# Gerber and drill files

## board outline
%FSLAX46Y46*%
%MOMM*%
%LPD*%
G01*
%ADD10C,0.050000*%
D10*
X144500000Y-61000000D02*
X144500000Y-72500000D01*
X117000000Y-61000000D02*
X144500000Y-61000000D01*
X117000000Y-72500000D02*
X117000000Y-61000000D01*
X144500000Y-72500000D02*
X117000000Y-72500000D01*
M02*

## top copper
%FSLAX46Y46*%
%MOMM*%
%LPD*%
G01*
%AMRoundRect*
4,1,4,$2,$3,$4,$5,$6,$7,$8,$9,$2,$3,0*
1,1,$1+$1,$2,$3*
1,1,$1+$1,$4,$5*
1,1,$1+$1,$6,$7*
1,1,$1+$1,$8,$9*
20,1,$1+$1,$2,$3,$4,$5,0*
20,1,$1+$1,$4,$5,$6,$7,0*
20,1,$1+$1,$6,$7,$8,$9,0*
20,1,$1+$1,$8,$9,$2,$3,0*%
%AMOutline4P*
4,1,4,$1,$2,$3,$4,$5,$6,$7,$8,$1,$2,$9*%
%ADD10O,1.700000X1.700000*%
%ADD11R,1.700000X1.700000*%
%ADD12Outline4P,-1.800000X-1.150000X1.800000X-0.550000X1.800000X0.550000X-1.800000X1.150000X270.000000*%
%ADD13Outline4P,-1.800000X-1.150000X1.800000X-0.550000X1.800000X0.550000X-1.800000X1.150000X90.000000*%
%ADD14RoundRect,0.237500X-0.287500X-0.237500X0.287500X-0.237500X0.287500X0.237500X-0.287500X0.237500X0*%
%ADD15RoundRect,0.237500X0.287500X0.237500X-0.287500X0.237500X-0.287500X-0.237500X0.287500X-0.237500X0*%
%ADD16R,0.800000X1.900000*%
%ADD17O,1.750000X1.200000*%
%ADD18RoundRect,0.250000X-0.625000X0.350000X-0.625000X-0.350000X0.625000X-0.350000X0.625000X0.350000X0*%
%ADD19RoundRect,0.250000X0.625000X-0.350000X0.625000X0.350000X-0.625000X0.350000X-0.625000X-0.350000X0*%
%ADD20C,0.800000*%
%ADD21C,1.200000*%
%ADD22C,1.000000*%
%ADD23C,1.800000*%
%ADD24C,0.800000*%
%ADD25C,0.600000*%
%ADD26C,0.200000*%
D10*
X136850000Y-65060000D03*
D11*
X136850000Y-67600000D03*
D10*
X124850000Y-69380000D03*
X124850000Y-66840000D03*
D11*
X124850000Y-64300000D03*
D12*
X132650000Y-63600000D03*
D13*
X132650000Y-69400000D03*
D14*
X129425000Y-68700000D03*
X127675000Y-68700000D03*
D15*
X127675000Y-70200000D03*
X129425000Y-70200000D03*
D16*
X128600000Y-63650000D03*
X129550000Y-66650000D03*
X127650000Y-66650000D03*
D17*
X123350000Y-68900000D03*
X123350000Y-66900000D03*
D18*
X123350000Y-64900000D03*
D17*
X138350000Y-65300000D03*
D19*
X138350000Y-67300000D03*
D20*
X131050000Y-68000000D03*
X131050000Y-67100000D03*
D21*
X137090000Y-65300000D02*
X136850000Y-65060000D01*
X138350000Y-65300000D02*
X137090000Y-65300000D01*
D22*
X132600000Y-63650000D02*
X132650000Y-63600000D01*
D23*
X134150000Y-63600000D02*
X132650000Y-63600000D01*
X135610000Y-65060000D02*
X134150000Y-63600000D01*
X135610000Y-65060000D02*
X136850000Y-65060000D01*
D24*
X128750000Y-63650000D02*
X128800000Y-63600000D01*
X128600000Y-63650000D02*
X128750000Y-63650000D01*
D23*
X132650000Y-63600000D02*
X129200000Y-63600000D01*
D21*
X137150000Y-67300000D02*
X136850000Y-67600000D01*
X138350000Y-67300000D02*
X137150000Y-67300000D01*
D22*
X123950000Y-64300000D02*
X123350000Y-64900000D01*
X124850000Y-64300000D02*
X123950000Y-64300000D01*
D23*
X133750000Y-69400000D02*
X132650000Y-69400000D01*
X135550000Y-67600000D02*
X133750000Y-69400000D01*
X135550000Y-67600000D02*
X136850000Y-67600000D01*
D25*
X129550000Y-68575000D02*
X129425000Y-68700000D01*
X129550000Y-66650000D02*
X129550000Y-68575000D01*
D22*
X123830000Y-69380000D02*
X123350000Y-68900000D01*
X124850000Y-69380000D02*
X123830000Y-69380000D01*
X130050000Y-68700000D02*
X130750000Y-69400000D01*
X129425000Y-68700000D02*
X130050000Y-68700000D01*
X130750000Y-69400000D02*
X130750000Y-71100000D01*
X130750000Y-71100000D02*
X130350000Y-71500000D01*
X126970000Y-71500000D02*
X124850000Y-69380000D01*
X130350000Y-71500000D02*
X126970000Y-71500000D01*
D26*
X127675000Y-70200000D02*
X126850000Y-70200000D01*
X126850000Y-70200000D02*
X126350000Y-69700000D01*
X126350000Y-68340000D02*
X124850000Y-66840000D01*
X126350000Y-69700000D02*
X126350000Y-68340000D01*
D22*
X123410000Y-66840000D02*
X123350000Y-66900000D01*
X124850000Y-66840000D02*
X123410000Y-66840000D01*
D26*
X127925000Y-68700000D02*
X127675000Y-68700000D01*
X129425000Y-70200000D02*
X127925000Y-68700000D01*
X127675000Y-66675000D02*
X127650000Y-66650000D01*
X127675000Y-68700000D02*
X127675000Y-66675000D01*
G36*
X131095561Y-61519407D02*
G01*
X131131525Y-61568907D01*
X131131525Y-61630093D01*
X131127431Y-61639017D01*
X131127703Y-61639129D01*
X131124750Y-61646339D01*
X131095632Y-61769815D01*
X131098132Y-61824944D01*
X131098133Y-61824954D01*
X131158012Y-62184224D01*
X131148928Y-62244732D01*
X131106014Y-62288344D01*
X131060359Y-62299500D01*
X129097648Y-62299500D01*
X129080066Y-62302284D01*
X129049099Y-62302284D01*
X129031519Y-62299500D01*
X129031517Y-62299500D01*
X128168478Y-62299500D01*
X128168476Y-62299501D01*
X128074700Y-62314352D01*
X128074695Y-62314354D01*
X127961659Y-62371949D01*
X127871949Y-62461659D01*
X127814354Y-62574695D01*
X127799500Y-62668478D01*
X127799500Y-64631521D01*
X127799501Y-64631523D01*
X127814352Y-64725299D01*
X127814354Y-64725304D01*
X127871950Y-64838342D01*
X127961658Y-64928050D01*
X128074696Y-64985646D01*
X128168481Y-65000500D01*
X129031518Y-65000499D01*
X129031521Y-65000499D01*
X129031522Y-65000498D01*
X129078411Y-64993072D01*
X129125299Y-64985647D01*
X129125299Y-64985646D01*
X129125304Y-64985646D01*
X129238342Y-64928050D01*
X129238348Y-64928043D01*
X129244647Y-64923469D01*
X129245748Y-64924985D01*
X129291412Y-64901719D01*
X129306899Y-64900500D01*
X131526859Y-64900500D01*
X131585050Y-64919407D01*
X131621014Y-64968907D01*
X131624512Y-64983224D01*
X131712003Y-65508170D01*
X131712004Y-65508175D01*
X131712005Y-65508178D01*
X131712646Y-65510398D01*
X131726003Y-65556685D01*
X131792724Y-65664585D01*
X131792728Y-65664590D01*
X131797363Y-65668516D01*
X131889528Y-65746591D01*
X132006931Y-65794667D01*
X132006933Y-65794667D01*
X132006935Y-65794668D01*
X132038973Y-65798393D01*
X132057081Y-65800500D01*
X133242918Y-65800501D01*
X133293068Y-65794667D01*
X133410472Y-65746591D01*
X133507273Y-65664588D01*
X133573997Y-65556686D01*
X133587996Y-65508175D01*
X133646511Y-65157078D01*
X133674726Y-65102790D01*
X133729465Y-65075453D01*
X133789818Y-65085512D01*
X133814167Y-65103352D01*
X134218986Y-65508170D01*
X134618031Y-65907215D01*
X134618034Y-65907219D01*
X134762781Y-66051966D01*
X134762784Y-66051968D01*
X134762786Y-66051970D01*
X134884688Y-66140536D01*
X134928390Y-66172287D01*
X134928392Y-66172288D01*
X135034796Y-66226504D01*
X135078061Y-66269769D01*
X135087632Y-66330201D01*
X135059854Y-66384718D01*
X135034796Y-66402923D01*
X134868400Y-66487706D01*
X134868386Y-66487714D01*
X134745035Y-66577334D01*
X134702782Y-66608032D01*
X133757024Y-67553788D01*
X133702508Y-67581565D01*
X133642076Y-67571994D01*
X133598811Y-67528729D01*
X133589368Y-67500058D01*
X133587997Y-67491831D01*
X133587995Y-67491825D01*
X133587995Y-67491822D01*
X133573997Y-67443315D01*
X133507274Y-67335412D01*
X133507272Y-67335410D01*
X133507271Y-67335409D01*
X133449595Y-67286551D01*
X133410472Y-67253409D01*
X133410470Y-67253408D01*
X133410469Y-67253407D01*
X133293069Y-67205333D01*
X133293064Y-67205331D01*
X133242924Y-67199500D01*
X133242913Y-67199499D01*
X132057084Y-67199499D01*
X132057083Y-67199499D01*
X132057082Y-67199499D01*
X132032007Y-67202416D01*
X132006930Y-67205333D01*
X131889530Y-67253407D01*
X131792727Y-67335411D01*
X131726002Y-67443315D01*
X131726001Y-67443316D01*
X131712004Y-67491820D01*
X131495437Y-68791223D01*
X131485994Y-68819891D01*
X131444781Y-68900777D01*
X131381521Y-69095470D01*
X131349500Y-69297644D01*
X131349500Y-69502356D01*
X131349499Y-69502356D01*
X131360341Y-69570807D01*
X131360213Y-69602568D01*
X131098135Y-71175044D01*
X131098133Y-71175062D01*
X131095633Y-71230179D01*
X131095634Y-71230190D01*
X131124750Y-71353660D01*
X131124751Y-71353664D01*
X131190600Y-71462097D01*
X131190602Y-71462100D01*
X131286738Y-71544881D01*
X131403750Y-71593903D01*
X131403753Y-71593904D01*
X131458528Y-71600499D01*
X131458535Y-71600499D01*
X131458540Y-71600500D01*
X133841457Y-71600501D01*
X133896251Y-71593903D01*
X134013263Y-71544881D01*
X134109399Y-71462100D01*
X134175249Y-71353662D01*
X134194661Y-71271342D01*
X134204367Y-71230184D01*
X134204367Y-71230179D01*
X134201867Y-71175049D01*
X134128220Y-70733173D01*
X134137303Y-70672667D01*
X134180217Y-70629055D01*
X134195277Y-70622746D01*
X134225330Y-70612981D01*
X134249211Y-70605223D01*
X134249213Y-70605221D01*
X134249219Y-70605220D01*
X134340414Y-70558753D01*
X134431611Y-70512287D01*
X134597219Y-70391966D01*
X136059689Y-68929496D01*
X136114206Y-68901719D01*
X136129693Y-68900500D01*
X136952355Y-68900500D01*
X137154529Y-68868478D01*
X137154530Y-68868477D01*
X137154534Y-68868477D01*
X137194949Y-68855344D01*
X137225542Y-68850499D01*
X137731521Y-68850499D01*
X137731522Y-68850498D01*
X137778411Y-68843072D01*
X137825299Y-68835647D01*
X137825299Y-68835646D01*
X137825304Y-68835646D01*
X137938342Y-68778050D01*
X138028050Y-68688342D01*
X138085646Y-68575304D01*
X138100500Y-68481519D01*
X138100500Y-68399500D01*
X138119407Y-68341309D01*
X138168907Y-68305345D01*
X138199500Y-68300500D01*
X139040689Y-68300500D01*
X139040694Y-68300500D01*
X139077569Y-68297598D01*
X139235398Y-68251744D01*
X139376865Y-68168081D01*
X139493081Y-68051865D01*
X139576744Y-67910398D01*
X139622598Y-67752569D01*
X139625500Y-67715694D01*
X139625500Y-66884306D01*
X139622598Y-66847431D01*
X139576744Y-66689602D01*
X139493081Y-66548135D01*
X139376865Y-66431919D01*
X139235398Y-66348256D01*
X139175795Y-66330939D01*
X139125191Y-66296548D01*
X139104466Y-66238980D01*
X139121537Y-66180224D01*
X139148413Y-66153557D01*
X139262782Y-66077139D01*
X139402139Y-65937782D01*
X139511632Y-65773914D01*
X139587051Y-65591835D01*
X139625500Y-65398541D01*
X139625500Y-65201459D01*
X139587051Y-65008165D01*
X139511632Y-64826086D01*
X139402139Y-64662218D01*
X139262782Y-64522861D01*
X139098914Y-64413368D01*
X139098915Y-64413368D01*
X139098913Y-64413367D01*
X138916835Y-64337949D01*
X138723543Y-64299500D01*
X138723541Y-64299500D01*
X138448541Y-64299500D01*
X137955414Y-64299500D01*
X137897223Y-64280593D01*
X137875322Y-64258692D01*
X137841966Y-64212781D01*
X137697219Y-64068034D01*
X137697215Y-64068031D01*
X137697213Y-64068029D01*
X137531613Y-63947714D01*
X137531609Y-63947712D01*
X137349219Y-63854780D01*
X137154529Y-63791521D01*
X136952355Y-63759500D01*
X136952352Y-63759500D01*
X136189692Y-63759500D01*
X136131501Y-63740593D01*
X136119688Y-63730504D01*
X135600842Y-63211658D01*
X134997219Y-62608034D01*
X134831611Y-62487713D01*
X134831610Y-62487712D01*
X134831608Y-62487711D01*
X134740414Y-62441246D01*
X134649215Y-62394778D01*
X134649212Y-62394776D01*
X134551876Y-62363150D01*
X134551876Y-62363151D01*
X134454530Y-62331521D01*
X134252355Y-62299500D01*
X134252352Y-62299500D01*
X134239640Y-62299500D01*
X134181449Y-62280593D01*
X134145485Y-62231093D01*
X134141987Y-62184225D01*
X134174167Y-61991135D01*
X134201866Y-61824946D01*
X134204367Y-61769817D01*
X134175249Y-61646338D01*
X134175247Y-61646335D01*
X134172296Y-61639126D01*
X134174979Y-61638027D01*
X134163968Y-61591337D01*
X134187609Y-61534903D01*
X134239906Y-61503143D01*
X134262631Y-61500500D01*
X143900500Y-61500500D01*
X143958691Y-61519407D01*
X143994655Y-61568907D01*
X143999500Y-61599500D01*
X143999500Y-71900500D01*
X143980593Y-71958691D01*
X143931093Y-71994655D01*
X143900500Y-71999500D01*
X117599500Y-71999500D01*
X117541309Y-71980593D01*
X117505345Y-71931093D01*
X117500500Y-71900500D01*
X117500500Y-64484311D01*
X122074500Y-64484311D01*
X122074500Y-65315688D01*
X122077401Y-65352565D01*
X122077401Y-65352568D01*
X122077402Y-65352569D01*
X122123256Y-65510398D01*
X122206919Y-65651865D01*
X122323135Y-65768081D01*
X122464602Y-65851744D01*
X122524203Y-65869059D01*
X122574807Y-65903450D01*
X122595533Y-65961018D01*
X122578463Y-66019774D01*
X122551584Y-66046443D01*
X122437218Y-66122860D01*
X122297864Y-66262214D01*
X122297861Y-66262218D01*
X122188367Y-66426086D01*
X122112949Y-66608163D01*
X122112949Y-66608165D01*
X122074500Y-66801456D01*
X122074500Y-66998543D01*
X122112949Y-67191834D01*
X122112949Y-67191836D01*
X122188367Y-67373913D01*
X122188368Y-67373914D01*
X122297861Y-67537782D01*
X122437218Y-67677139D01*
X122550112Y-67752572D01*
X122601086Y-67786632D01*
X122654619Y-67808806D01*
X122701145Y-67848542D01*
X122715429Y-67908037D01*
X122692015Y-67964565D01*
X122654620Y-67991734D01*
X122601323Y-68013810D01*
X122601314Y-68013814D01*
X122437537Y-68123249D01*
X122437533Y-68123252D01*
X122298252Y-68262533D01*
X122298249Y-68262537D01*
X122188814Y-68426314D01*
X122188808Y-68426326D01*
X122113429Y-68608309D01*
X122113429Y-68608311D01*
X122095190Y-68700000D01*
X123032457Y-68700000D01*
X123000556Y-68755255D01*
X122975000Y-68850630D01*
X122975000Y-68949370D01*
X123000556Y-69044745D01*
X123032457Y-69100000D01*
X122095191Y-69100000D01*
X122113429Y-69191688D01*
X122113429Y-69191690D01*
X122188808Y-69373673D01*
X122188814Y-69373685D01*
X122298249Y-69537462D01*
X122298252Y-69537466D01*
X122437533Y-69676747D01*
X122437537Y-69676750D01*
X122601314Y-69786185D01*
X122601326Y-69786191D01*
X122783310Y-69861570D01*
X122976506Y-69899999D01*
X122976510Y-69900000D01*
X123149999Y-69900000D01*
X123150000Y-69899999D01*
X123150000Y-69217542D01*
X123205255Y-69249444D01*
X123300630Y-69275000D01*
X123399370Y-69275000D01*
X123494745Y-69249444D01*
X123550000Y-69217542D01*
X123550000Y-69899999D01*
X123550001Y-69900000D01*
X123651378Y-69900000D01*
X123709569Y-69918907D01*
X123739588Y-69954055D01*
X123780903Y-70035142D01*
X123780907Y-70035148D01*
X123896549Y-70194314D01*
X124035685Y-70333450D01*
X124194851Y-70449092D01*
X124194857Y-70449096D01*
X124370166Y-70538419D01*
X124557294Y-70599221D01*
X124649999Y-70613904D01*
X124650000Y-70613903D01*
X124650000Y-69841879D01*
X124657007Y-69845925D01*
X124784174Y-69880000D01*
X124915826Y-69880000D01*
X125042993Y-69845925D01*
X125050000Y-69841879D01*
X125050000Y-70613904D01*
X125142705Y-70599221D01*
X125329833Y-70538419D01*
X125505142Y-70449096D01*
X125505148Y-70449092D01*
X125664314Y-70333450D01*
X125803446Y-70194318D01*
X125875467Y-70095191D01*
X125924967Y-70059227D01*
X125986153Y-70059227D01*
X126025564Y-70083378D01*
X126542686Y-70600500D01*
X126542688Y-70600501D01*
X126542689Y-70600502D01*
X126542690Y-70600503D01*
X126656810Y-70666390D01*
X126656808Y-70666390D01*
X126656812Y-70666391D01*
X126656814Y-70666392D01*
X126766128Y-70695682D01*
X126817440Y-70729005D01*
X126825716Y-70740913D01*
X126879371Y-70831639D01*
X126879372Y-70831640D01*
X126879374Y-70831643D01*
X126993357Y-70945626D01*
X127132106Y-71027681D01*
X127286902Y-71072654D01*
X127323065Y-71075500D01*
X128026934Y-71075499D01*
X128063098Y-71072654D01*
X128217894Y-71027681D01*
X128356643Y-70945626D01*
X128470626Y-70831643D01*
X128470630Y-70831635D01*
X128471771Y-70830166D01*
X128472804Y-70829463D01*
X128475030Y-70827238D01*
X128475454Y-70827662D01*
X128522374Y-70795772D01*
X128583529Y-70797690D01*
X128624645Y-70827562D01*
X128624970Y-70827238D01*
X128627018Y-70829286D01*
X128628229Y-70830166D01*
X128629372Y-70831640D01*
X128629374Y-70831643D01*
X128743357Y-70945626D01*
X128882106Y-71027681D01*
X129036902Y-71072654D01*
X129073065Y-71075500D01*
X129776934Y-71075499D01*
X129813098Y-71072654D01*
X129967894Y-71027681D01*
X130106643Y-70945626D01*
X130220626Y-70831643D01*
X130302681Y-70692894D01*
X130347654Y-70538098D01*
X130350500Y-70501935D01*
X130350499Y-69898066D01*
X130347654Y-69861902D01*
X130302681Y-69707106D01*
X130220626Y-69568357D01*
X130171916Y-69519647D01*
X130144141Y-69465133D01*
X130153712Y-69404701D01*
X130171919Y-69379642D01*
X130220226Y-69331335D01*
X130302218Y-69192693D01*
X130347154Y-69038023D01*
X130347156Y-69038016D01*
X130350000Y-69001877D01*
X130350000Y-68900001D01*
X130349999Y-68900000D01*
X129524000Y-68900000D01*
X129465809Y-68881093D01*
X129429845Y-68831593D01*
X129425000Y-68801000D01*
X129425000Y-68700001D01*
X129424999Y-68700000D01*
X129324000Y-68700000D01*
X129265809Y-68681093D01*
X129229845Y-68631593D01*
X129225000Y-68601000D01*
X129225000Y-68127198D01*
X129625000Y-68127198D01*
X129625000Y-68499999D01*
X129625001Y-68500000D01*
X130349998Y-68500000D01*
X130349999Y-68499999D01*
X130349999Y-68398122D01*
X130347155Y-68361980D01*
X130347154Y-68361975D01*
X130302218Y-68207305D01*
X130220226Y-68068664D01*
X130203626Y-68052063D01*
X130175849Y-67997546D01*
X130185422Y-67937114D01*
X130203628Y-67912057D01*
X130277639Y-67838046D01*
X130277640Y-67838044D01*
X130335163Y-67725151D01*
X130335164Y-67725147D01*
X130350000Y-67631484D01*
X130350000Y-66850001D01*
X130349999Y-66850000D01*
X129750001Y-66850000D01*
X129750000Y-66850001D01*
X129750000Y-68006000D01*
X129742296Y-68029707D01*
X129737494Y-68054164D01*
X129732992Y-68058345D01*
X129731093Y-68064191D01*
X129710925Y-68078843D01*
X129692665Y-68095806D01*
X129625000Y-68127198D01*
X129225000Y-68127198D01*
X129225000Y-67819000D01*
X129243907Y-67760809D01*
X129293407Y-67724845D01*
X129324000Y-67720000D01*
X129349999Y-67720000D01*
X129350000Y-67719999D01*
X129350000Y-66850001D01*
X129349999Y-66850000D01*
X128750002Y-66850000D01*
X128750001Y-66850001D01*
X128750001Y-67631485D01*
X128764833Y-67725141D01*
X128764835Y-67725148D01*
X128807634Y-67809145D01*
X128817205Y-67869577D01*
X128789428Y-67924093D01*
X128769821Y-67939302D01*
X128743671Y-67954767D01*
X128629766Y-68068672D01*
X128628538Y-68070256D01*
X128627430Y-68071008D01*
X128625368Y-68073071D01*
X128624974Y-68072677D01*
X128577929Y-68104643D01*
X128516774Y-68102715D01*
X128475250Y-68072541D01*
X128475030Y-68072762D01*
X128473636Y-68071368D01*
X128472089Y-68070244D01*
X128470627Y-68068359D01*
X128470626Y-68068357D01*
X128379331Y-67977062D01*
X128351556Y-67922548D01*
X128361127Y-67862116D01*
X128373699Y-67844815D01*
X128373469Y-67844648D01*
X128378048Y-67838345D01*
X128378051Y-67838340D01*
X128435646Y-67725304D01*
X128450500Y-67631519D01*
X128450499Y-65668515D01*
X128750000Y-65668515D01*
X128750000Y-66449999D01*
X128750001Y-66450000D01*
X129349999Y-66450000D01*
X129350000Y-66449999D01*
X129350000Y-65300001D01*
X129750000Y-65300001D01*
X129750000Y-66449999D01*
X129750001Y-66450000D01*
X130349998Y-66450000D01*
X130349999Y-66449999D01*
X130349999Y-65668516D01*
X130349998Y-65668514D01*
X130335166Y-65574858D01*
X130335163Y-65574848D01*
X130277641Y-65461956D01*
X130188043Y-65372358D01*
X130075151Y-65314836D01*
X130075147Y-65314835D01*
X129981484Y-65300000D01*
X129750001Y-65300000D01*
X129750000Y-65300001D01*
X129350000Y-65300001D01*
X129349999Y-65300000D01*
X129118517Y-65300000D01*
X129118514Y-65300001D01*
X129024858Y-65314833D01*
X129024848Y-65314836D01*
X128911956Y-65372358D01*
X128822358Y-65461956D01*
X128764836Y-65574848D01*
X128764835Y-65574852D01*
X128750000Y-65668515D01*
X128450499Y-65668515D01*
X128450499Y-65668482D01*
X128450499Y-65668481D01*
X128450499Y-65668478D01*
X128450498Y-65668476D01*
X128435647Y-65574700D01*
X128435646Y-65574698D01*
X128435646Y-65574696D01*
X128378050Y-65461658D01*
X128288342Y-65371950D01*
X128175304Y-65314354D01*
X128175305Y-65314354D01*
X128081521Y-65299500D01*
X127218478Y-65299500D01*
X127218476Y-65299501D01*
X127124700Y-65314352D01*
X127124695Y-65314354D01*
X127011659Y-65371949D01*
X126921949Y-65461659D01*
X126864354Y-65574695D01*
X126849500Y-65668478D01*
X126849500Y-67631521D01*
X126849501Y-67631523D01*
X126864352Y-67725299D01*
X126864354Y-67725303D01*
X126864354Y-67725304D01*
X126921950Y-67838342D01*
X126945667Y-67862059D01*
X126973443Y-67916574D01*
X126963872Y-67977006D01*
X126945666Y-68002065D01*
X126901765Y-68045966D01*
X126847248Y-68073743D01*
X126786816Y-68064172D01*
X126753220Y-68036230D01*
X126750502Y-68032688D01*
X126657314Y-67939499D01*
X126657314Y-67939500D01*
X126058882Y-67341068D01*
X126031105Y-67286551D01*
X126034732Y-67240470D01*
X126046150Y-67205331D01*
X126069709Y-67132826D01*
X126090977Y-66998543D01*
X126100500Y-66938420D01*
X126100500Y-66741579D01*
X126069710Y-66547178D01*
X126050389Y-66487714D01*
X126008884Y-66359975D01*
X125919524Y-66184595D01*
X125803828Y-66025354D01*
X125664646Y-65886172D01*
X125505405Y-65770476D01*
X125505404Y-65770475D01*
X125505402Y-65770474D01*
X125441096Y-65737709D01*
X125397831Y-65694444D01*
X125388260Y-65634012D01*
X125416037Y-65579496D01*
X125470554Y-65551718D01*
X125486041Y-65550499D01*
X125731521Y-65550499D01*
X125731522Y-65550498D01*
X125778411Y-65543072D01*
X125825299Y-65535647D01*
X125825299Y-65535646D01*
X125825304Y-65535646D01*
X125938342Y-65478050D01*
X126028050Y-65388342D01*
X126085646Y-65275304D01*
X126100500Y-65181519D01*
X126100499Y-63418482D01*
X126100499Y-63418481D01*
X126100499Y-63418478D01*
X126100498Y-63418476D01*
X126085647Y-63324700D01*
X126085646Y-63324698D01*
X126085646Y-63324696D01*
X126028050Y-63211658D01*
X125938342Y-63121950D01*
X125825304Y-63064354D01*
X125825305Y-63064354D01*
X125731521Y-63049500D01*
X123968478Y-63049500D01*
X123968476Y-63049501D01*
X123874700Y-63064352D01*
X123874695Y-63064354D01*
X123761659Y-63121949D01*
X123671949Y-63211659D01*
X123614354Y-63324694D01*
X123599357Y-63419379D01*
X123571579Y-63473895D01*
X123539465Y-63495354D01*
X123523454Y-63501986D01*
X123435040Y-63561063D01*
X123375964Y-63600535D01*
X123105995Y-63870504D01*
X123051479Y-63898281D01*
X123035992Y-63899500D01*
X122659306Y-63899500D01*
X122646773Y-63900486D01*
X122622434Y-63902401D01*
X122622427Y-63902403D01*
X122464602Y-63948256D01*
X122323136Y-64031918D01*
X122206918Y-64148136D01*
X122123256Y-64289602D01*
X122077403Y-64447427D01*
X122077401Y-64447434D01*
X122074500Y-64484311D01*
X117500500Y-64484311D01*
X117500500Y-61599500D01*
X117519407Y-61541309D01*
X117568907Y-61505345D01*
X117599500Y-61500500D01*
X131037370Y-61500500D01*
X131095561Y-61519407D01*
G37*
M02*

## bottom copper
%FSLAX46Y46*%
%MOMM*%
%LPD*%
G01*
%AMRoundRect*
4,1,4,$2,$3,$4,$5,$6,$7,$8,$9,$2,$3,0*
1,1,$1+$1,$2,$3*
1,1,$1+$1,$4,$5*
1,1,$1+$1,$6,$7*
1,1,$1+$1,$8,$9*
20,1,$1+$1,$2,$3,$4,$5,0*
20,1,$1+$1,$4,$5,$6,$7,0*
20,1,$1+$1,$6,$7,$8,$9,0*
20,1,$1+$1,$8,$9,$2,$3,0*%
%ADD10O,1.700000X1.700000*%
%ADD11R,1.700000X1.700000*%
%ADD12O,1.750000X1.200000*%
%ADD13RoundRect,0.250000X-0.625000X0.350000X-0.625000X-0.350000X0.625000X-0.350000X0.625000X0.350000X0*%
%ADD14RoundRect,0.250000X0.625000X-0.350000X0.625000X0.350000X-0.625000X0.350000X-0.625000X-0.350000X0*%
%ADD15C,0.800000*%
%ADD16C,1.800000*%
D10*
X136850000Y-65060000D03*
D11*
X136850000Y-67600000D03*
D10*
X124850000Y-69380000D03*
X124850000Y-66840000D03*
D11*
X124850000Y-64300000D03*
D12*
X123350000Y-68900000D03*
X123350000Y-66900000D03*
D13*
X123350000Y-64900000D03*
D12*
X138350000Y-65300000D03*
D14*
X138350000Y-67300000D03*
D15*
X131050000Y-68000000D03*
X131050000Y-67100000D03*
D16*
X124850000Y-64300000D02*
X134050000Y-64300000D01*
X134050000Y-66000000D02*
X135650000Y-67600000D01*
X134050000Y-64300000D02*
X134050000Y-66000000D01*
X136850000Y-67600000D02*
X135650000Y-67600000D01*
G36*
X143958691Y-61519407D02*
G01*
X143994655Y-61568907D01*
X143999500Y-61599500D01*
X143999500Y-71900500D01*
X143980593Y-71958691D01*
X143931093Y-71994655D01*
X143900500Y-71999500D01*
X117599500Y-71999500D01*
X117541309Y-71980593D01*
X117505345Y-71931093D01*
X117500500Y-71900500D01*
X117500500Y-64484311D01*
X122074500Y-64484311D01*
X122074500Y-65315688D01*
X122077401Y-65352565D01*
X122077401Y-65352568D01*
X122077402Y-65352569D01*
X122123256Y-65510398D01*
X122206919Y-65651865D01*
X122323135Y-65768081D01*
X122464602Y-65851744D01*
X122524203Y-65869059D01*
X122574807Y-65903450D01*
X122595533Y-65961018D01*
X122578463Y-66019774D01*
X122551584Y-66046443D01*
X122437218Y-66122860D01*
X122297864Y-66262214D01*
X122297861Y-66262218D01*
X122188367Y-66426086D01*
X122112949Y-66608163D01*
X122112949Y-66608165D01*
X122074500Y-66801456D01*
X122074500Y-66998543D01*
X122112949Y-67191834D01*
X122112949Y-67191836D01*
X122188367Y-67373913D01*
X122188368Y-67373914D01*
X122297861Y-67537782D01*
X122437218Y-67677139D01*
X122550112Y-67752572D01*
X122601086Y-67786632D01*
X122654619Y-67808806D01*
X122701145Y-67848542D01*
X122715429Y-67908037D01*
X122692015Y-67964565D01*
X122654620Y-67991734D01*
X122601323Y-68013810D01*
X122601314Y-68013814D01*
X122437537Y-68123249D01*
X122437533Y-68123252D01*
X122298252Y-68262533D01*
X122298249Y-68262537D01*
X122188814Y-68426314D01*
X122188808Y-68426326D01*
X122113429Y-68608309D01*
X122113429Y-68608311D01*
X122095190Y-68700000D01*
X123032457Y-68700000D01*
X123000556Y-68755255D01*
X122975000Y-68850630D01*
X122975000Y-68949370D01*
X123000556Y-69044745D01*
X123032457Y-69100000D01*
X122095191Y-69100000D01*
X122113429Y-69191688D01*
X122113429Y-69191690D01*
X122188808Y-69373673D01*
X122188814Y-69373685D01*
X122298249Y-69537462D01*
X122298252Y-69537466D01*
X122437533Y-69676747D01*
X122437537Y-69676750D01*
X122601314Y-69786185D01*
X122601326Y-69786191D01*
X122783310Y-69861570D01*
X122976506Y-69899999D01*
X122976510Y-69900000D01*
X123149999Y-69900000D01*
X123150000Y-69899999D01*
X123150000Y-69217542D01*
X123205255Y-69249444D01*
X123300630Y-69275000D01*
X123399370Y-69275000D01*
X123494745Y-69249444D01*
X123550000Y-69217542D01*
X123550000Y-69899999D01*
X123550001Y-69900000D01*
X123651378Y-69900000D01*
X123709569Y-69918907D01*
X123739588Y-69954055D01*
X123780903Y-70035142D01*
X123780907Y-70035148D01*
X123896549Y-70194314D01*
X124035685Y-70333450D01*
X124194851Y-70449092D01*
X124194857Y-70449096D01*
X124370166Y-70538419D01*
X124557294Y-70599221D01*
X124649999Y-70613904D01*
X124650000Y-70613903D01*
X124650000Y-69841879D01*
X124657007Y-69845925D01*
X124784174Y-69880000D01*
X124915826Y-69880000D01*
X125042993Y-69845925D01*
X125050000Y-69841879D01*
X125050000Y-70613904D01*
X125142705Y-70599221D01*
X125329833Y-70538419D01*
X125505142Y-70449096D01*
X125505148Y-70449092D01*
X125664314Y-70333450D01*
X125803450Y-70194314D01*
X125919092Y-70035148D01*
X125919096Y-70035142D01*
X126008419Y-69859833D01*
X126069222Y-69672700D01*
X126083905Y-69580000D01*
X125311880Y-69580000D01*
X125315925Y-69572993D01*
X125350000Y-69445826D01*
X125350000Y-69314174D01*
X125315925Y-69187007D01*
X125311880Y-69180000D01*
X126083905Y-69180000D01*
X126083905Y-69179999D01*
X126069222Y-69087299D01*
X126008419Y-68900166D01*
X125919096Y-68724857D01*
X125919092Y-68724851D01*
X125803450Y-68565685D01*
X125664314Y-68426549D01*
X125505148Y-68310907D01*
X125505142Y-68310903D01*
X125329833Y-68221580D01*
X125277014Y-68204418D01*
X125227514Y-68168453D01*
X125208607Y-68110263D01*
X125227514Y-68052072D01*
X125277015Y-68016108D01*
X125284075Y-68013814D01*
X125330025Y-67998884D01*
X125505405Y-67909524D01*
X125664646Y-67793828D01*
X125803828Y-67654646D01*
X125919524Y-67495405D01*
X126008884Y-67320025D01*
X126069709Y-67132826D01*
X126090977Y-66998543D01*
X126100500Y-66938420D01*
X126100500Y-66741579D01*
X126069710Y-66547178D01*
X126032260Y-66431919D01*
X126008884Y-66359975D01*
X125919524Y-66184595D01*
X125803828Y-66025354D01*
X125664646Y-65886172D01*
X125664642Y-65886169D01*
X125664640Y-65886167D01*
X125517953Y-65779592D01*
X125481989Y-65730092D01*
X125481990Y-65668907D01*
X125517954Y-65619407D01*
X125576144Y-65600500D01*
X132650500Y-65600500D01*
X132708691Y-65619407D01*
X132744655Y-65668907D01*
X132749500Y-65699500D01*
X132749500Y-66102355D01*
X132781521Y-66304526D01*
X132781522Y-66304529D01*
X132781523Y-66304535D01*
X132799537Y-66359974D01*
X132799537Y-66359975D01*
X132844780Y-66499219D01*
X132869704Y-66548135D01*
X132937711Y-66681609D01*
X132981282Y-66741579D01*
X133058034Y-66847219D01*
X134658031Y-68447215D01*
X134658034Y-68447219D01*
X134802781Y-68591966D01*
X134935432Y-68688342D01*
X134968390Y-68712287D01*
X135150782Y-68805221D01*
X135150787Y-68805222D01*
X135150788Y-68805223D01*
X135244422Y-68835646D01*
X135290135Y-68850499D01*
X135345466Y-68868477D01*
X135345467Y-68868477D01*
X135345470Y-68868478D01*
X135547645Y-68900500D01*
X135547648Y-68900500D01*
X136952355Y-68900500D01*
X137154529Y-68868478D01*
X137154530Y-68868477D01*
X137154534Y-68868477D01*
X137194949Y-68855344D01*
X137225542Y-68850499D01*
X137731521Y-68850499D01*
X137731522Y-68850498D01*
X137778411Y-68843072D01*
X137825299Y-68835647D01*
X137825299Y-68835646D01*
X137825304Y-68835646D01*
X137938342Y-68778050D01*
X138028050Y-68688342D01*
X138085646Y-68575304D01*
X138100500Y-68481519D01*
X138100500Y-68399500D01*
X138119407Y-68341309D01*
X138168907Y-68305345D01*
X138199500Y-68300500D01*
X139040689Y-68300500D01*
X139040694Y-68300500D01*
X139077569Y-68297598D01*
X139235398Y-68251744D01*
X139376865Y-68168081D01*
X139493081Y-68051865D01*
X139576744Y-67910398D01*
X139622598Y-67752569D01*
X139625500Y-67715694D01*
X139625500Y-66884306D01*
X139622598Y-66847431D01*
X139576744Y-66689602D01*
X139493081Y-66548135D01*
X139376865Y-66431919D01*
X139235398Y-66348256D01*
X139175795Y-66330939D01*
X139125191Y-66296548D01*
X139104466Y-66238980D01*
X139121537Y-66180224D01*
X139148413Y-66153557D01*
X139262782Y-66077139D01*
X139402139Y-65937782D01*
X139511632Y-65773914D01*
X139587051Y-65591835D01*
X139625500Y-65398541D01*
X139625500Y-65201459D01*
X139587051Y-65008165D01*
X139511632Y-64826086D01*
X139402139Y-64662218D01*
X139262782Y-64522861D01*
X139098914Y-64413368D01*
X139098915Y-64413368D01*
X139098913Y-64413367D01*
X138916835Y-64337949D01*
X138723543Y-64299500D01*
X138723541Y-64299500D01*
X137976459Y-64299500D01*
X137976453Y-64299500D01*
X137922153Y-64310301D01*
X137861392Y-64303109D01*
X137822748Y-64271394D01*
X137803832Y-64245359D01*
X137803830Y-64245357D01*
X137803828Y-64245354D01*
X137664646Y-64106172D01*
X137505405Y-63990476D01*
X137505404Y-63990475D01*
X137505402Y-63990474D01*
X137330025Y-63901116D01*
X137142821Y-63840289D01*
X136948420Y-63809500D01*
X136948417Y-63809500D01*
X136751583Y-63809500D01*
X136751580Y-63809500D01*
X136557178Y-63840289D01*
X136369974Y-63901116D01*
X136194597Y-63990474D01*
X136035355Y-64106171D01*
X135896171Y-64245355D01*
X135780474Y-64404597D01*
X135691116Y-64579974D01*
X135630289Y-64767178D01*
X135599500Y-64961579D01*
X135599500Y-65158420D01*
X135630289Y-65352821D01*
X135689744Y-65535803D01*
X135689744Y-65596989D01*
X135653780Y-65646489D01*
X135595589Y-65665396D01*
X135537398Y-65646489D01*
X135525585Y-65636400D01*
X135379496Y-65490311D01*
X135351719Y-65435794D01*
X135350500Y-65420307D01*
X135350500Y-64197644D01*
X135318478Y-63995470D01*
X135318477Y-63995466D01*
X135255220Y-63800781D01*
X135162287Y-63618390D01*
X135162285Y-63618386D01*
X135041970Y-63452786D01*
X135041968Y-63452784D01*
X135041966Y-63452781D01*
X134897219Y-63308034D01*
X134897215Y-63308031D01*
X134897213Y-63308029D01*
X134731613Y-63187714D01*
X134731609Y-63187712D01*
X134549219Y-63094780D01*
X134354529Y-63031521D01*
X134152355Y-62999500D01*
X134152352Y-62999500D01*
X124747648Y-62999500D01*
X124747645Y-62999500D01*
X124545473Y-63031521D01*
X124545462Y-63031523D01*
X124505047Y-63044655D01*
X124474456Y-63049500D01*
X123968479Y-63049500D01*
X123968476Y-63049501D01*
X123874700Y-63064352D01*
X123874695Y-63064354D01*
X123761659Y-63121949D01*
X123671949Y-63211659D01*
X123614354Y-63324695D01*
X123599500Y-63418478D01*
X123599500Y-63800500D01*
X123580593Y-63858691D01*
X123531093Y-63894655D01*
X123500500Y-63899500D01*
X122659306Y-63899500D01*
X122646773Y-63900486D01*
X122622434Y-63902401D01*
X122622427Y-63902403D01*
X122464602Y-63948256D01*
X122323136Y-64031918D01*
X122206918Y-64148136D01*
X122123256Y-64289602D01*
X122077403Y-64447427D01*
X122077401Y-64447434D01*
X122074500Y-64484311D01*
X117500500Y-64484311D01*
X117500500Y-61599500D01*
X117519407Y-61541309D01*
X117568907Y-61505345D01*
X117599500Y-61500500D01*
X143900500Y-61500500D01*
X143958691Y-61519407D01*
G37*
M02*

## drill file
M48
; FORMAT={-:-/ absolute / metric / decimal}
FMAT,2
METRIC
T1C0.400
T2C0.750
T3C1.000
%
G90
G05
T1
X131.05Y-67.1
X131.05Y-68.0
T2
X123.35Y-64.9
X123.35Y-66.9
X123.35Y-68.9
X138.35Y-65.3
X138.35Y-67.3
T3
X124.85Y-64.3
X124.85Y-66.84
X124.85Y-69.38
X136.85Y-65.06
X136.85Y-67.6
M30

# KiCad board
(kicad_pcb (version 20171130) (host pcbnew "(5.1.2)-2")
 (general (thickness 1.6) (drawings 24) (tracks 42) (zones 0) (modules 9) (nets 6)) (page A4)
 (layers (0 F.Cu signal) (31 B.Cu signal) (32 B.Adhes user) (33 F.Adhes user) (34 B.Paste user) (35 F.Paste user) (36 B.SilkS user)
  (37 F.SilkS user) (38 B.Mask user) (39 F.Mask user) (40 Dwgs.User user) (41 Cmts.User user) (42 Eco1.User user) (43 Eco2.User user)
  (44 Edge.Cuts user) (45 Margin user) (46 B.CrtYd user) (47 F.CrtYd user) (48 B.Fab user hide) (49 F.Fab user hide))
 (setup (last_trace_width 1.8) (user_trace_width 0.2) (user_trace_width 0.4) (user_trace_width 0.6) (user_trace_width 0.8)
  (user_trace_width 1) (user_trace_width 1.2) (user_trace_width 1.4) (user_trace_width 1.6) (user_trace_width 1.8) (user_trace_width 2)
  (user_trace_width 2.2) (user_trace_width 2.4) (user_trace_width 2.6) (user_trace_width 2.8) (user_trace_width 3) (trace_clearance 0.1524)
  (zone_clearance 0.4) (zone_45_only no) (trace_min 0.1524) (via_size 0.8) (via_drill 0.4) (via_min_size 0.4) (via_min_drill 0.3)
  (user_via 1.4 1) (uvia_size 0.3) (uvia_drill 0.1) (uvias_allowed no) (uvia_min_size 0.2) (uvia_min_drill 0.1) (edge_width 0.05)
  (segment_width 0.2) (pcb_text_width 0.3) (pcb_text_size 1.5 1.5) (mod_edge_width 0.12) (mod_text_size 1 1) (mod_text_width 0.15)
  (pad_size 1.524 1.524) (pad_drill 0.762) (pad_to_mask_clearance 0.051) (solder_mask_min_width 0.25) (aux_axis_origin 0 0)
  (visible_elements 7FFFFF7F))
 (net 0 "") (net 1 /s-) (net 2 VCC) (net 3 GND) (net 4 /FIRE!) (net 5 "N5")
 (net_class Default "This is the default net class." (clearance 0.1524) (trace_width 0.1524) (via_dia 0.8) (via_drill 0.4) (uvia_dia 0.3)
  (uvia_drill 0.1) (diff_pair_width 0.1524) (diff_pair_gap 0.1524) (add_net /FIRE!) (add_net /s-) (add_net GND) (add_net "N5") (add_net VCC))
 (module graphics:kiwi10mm (layer B.Cu) (at 131 66.8 270)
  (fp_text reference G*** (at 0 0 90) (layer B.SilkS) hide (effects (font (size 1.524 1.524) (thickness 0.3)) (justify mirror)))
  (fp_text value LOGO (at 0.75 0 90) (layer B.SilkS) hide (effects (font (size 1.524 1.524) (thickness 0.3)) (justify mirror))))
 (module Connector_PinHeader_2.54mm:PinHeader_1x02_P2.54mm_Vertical (layer F.Cu) (at 136.85 67.6 180)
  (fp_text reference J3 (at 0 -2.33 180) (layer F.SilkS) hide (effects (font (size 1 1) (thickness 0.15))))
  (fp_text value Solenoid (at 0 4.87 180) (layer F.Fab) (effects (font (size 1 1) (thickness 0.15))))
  (pad 2 thru_hole oval (at 0 2.54 180) (size 1.7 1.7) (drill 1) (layers *.Cu *.Mask) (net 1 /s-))
  (pad 1 thru_hole rect (at 0 0 180) (size 1.7 1.7) (drill 1) (layers *.Cu *.Mask) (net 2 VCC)))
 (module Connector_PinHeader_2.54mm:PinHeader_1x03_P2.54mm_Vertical (layer F.Cu) (at 124.85 64.3)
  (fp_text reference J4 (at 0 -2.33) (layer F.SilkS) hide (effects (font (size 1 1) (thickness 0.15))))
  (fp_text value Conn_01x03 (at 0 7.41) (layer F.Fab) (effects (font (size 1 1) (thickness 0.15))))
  (pad 3 thru_hole oval (at 0 5.08) (size 1.7 1.7) (drill 1) (layers *.Cu *.Mask) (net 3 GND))
  (pad 2 thru_hole oval (at 0 2.54) (size 1.7 1.7) (drill 1) (layers *.Cu *.Mask) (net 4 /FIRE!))
  (pad 1 thru_hole rect (at 0 0) (size 1.7 1.7) (drill 1) (layers *.Cu *.Mask) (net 2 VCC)))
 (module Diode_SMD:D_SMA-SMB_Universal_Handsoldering (layer F.Cu) (at 132.65 66.5 90)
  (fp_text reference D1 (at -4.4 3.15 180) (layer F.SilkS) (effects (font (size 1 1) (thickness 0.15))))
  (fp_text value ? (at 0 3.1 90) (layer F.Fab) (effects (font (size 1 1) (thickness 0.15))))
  (pad 2 smd trapezoid (at 2.9 0 270) (size 3.6 1.7) (rect_delta 0.6 0) (layers F.Cu F.Paste F.Mask) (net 1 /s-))
  (pad 1 smd trapezoid (at -2.9 0 90) (size 3.6 1.7) (rect_delta 0.6 0) (layers F.Cu F.Paste F.Mask) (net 2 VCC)))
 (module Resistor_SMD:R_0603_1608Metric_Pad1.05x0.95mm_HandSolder (layer F.Cu) (at 128.55 68.7)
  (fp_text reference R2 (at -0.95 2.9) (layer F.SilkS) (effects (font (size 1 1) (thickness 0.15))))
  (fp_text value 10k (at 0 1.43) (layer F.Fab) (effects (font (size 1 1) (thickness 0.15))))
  (pad 2 smd roundrect (at 0.875 0) (size 1.05 0.95) (layers F.Cu F.Paste F.Mask) (roundrect_rratio 0.25) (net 3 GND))
  (pad 1 smd roundrect (at -0.875 0) (size 1.05 0.95) (layers F.Cu F.Paste F.Mask) (roundrect_rratio 0.25) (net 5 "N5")))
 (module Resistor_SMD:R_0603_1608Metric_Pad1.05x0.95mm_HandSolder (layer F.Cu) (at 128.55 70.2 180)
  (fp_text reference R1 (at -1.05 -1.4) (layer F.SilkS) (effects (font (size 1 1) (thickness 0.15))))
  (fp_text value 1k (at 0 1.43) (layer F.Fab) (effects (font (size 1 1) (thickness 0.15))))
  (pad 2 smd roundrect (at 0.875 0 180) (size 1.05 0.95) (layers F.Cu F.Paste F.Mask) (roundrect_rratio 0.25) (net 4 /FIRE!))
  (pad 1 smd roundrect (at -0.875 0 180) (size 1.05 0.95) (layers F.Cu F.Paste F.Mask) (roundrect_rratio 0.25) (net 5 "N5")))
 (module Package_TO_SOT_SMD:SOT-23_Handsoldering (layer F.Cu) (at 128.6 65.15 90)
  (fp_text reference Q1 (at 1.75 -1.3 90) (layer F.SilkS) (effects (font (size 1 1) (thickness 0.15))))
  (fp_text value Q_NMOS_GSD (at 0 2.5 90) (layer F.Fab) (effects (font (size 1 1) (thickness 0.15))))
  (pad 3 smd rect (at 1.5 0 90) (size 1.9 0.8) (layers F.Cu F.Paste F.Mask) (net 1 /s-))
  (pad 2 smd rect (at -1.5 0.95 90) (size 1.9 0.8) (layers F.Cu F.Paste F.Mask) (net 3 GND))
  (pad 1 smd rect (at -1.5 -0.95 90) (size 1.9 0.8) (layers F.Cu F.Paste F.Mask) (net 5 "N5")))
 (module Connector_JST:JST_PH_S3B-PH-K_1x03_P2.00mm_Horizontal (layer F.Cu) (at 123.35 64.9 270)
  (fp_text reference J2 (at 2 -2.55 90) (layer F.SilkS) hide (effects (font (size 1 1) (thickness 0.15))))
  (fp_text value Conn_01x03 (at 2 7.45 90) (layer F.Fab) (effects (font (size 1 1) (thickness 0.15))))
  (pad 3 thru_hole oval (at 4 0 270) (size 1.2 1.75) (drill 0.75) (layers *.Cu *.Mask) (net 3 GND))
  (pad 2 thru_hole oval (at 2 0 270) (size 1.2 1.75) (drill 0.75) (layers *.Cu *.Mask) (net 4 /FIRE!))
  (pad 1 thru_hole roundrect (at 0 0 270) (size 1.2 1.75) (drill 0.75) (layers *.Cu *.Mask) (roundrect_rratio 0.208333) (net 2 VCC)))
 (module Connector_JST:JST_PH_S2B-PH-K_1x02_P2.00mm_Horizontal (layer F.Cu) (at 138.35 67.3 90)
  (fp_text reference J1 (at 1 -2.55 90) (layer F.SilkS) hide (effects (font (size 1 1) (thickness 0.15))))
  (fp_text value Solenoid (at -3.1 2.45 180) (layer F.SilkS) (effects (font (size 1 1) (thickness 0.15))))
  (pad 2 thru_hole oval (at 2 0 90) (size 1.2 1.75) (drill 0.75) (layers *.Cu *.Mask) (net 1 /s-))
  (pad 1 thru_hole roundrect (at 0 0 90) (size 1.2 1.75) (drill 0.75) (layers *.Cu *.Mask) (roundrect_rratio 0.208333) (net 2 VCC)))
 (gr_line (start 144.5 61) (end 144.5 72.5) (layer Edge.Cuts) (width 0.05))
 (gr_line (start 117 61) (end 144.5 61) (layer Edge.Cuts) (width 0.05))
 (gr_line (start 117 72.5) (end 117 61) (layer Edge.Cuts) (width 0.05))
 (gr_line (start 144.5 72.5) (end 117 72.5) (layer Edge.Cuts) (width 0.05))
 (via (at 131.05 68) (size 0.8) (drill 0.4) (layers F.Cu B.Cu) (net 3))
 (via (at 131.05 67.1) (size 0.8) (drill 0.4) (layers F.Cu B.Cu) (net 3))
 (segment (start 137.09 65.3) (end 136.85 65.06) (width 1.2) (layer F.Cu) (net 1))
 (segment (start 138.35 65.3) (end 137.09 65.3) (width 1.2) (layer F.Cu) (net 1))
 (segment (start 132.6 63.65) (end 132.65 63.6) (width 1) (layer F.Cu) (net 1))
 (segment (start 134.15 63.6) (end 132.65 63.6) (width 1.8) (layer F.Cu) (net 1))
 (segment (start 135.61 65.06) (end 134.15 63.6) (width 1.8) (layer F.Cu) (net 1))
 (segment (start 135.61 65.06) (end 136.85 65.06) (width 1.8) (layer F.Cu) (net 1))
 (segment (start 128.75 63.65) (end 128.8 63.6) (width 0.8) (layer F.Cu) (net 1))
 (segment (start 128.6 63.65) (end 128.75 63.65) (width 0.8) (layer F.Cu) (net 1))
 (segment (start 132.65 63.6) (end 129.2 63.6) (width 1.8) (layer F.Cu) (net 1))
 (segment (start 137.15 67.3) (end 136.85 67.6) (width 1.2) (layer F.Cu) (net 2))
 (segment (start 138.35 67.3) (end 137.15 67.3) (width 1.2) (layer F.Cu) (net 2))
 (segment (start 123.95 64.3) (end 123.35 64.9) (width 1) (layer F.Cu) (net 2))
 (segment (start 124.85 64.3) (end 123.95 64.3) (width 1) (layer F.Cu) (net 2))
 (segment (start 133.75 69.4) (end 132.65 69.4) (width 1.8) (layer F.Cu) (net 2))
 (segment (start 135.55 67.6) (end 133.75 69.4) (width 1.8) (layer F.Cu) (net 2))
 (segment (start 135.55 67.6) (end 136.85 67.6) (width 1.8) (layer F.Cu) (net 2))
 (segment (start 124.85 64.3) (end 134.05 64.3) (width 1.8) (layer B.Cu) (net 2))
 (segment (start 134.05 66) (end 135.65 67.6) (width 1.8) (layer B.Cu) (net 2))
 (segment (start 134.05 64.3) (end 134.05 66) (width 1.8) (layer B.Cu) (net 2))
 (segment (start 136.85 67.6) (end 135.65 67.6) (width 1.8) (layer B.Cu) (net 2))
 (segment (start 129.55 68.575) (end 129.425 68.7) (width 0.6) (layer F.Cu) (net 3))
 (segment (start 129.55 66.65) (end 129.55 68.575) (width 0.6) (layer F.Cu) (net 3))
 (segment (start 123.83 69.38) (end 123.35 68.9) (width 1) (layer F.Cu) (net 3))
 (segment (start 124.85 69.38) (end 123.83 69.38) (width 1) (layer F.Cu) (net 3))
 (segment (start 130.05 68.7) (end 130.75 69.4) (width 1) (layer F.Cu) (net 3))
 (segment (start 129.425 68.7) (end 130.05 68.7) (width 1) (layer F.Cu) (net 3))
 (segment (start 130.75 69.4) (end 130.75 71.1) (width 1) (layer F.Cu) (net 3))
 (segment (start 130.75 71.1) (end 130.35 71.5) (width 1) (layer F.Cu) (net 3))
 (segment (start 126.97 71.5) (end 124.85 69.38) (width 1) (layer F.Cu) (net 3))
 (segment (start 130.35 71.5) (end 126.97 71.5) (width 1) (layer F.Cu) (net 3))
 (segment (start 127.675 70.2) (end 126.85 70.2) (width 0.2) (layer F.Cu) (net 4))
 (segment (start 126.85 70.2) (end 126.35 69.7) (width 0.2) (layer F.Cu) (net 4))
 (segment (start 126.35 68.34) (end 124.85 66.84) (width 0.2) (layer F.Cu) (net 4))
 (segment (start 126.35 69.7) (end 126.35 68.34) (width 0.2) (layer F.Cu) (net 4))
 (segment (start 123.41 66.84) (end 123.35 66.9) (width 1) (layer F.Cu) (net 4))
 (segment (start 124.85 66.84) (end 123.41 66.84) (width 1) (layer F.Cu) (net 4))
 (segment (start 127.925 68.7) (end 127.675 68.7) (width 0.2) (layer F.Cu) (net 5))
 (segment (start 129.425 70.2) (end 127.925 68.7) (width 0.2) (layer F.Cu) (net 5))
 (segment (start 127.675 66.675) (end 127.65 66.65) (width 0.2) (layer F.Cu) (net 5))
 (segment (start 127.675 68.7) (end 127.675 66.675) (width 0.2) (layer F.Cu) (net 5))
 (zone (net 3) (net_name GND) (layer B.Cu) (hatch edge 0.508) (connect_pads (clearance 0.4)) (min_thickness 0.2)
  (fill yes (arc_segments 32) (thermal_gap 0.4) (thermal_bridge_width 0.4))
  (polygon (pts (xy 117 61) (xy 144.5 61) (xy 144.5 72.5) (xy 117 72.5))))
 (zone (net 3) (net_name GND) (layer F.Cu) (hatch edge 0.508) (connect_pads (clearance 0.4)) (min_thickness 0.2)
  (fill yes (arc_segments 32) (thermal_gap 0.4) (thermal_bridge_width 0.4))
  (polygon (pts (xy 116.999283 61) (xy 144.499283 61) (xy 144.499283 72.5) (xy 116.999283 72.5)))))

